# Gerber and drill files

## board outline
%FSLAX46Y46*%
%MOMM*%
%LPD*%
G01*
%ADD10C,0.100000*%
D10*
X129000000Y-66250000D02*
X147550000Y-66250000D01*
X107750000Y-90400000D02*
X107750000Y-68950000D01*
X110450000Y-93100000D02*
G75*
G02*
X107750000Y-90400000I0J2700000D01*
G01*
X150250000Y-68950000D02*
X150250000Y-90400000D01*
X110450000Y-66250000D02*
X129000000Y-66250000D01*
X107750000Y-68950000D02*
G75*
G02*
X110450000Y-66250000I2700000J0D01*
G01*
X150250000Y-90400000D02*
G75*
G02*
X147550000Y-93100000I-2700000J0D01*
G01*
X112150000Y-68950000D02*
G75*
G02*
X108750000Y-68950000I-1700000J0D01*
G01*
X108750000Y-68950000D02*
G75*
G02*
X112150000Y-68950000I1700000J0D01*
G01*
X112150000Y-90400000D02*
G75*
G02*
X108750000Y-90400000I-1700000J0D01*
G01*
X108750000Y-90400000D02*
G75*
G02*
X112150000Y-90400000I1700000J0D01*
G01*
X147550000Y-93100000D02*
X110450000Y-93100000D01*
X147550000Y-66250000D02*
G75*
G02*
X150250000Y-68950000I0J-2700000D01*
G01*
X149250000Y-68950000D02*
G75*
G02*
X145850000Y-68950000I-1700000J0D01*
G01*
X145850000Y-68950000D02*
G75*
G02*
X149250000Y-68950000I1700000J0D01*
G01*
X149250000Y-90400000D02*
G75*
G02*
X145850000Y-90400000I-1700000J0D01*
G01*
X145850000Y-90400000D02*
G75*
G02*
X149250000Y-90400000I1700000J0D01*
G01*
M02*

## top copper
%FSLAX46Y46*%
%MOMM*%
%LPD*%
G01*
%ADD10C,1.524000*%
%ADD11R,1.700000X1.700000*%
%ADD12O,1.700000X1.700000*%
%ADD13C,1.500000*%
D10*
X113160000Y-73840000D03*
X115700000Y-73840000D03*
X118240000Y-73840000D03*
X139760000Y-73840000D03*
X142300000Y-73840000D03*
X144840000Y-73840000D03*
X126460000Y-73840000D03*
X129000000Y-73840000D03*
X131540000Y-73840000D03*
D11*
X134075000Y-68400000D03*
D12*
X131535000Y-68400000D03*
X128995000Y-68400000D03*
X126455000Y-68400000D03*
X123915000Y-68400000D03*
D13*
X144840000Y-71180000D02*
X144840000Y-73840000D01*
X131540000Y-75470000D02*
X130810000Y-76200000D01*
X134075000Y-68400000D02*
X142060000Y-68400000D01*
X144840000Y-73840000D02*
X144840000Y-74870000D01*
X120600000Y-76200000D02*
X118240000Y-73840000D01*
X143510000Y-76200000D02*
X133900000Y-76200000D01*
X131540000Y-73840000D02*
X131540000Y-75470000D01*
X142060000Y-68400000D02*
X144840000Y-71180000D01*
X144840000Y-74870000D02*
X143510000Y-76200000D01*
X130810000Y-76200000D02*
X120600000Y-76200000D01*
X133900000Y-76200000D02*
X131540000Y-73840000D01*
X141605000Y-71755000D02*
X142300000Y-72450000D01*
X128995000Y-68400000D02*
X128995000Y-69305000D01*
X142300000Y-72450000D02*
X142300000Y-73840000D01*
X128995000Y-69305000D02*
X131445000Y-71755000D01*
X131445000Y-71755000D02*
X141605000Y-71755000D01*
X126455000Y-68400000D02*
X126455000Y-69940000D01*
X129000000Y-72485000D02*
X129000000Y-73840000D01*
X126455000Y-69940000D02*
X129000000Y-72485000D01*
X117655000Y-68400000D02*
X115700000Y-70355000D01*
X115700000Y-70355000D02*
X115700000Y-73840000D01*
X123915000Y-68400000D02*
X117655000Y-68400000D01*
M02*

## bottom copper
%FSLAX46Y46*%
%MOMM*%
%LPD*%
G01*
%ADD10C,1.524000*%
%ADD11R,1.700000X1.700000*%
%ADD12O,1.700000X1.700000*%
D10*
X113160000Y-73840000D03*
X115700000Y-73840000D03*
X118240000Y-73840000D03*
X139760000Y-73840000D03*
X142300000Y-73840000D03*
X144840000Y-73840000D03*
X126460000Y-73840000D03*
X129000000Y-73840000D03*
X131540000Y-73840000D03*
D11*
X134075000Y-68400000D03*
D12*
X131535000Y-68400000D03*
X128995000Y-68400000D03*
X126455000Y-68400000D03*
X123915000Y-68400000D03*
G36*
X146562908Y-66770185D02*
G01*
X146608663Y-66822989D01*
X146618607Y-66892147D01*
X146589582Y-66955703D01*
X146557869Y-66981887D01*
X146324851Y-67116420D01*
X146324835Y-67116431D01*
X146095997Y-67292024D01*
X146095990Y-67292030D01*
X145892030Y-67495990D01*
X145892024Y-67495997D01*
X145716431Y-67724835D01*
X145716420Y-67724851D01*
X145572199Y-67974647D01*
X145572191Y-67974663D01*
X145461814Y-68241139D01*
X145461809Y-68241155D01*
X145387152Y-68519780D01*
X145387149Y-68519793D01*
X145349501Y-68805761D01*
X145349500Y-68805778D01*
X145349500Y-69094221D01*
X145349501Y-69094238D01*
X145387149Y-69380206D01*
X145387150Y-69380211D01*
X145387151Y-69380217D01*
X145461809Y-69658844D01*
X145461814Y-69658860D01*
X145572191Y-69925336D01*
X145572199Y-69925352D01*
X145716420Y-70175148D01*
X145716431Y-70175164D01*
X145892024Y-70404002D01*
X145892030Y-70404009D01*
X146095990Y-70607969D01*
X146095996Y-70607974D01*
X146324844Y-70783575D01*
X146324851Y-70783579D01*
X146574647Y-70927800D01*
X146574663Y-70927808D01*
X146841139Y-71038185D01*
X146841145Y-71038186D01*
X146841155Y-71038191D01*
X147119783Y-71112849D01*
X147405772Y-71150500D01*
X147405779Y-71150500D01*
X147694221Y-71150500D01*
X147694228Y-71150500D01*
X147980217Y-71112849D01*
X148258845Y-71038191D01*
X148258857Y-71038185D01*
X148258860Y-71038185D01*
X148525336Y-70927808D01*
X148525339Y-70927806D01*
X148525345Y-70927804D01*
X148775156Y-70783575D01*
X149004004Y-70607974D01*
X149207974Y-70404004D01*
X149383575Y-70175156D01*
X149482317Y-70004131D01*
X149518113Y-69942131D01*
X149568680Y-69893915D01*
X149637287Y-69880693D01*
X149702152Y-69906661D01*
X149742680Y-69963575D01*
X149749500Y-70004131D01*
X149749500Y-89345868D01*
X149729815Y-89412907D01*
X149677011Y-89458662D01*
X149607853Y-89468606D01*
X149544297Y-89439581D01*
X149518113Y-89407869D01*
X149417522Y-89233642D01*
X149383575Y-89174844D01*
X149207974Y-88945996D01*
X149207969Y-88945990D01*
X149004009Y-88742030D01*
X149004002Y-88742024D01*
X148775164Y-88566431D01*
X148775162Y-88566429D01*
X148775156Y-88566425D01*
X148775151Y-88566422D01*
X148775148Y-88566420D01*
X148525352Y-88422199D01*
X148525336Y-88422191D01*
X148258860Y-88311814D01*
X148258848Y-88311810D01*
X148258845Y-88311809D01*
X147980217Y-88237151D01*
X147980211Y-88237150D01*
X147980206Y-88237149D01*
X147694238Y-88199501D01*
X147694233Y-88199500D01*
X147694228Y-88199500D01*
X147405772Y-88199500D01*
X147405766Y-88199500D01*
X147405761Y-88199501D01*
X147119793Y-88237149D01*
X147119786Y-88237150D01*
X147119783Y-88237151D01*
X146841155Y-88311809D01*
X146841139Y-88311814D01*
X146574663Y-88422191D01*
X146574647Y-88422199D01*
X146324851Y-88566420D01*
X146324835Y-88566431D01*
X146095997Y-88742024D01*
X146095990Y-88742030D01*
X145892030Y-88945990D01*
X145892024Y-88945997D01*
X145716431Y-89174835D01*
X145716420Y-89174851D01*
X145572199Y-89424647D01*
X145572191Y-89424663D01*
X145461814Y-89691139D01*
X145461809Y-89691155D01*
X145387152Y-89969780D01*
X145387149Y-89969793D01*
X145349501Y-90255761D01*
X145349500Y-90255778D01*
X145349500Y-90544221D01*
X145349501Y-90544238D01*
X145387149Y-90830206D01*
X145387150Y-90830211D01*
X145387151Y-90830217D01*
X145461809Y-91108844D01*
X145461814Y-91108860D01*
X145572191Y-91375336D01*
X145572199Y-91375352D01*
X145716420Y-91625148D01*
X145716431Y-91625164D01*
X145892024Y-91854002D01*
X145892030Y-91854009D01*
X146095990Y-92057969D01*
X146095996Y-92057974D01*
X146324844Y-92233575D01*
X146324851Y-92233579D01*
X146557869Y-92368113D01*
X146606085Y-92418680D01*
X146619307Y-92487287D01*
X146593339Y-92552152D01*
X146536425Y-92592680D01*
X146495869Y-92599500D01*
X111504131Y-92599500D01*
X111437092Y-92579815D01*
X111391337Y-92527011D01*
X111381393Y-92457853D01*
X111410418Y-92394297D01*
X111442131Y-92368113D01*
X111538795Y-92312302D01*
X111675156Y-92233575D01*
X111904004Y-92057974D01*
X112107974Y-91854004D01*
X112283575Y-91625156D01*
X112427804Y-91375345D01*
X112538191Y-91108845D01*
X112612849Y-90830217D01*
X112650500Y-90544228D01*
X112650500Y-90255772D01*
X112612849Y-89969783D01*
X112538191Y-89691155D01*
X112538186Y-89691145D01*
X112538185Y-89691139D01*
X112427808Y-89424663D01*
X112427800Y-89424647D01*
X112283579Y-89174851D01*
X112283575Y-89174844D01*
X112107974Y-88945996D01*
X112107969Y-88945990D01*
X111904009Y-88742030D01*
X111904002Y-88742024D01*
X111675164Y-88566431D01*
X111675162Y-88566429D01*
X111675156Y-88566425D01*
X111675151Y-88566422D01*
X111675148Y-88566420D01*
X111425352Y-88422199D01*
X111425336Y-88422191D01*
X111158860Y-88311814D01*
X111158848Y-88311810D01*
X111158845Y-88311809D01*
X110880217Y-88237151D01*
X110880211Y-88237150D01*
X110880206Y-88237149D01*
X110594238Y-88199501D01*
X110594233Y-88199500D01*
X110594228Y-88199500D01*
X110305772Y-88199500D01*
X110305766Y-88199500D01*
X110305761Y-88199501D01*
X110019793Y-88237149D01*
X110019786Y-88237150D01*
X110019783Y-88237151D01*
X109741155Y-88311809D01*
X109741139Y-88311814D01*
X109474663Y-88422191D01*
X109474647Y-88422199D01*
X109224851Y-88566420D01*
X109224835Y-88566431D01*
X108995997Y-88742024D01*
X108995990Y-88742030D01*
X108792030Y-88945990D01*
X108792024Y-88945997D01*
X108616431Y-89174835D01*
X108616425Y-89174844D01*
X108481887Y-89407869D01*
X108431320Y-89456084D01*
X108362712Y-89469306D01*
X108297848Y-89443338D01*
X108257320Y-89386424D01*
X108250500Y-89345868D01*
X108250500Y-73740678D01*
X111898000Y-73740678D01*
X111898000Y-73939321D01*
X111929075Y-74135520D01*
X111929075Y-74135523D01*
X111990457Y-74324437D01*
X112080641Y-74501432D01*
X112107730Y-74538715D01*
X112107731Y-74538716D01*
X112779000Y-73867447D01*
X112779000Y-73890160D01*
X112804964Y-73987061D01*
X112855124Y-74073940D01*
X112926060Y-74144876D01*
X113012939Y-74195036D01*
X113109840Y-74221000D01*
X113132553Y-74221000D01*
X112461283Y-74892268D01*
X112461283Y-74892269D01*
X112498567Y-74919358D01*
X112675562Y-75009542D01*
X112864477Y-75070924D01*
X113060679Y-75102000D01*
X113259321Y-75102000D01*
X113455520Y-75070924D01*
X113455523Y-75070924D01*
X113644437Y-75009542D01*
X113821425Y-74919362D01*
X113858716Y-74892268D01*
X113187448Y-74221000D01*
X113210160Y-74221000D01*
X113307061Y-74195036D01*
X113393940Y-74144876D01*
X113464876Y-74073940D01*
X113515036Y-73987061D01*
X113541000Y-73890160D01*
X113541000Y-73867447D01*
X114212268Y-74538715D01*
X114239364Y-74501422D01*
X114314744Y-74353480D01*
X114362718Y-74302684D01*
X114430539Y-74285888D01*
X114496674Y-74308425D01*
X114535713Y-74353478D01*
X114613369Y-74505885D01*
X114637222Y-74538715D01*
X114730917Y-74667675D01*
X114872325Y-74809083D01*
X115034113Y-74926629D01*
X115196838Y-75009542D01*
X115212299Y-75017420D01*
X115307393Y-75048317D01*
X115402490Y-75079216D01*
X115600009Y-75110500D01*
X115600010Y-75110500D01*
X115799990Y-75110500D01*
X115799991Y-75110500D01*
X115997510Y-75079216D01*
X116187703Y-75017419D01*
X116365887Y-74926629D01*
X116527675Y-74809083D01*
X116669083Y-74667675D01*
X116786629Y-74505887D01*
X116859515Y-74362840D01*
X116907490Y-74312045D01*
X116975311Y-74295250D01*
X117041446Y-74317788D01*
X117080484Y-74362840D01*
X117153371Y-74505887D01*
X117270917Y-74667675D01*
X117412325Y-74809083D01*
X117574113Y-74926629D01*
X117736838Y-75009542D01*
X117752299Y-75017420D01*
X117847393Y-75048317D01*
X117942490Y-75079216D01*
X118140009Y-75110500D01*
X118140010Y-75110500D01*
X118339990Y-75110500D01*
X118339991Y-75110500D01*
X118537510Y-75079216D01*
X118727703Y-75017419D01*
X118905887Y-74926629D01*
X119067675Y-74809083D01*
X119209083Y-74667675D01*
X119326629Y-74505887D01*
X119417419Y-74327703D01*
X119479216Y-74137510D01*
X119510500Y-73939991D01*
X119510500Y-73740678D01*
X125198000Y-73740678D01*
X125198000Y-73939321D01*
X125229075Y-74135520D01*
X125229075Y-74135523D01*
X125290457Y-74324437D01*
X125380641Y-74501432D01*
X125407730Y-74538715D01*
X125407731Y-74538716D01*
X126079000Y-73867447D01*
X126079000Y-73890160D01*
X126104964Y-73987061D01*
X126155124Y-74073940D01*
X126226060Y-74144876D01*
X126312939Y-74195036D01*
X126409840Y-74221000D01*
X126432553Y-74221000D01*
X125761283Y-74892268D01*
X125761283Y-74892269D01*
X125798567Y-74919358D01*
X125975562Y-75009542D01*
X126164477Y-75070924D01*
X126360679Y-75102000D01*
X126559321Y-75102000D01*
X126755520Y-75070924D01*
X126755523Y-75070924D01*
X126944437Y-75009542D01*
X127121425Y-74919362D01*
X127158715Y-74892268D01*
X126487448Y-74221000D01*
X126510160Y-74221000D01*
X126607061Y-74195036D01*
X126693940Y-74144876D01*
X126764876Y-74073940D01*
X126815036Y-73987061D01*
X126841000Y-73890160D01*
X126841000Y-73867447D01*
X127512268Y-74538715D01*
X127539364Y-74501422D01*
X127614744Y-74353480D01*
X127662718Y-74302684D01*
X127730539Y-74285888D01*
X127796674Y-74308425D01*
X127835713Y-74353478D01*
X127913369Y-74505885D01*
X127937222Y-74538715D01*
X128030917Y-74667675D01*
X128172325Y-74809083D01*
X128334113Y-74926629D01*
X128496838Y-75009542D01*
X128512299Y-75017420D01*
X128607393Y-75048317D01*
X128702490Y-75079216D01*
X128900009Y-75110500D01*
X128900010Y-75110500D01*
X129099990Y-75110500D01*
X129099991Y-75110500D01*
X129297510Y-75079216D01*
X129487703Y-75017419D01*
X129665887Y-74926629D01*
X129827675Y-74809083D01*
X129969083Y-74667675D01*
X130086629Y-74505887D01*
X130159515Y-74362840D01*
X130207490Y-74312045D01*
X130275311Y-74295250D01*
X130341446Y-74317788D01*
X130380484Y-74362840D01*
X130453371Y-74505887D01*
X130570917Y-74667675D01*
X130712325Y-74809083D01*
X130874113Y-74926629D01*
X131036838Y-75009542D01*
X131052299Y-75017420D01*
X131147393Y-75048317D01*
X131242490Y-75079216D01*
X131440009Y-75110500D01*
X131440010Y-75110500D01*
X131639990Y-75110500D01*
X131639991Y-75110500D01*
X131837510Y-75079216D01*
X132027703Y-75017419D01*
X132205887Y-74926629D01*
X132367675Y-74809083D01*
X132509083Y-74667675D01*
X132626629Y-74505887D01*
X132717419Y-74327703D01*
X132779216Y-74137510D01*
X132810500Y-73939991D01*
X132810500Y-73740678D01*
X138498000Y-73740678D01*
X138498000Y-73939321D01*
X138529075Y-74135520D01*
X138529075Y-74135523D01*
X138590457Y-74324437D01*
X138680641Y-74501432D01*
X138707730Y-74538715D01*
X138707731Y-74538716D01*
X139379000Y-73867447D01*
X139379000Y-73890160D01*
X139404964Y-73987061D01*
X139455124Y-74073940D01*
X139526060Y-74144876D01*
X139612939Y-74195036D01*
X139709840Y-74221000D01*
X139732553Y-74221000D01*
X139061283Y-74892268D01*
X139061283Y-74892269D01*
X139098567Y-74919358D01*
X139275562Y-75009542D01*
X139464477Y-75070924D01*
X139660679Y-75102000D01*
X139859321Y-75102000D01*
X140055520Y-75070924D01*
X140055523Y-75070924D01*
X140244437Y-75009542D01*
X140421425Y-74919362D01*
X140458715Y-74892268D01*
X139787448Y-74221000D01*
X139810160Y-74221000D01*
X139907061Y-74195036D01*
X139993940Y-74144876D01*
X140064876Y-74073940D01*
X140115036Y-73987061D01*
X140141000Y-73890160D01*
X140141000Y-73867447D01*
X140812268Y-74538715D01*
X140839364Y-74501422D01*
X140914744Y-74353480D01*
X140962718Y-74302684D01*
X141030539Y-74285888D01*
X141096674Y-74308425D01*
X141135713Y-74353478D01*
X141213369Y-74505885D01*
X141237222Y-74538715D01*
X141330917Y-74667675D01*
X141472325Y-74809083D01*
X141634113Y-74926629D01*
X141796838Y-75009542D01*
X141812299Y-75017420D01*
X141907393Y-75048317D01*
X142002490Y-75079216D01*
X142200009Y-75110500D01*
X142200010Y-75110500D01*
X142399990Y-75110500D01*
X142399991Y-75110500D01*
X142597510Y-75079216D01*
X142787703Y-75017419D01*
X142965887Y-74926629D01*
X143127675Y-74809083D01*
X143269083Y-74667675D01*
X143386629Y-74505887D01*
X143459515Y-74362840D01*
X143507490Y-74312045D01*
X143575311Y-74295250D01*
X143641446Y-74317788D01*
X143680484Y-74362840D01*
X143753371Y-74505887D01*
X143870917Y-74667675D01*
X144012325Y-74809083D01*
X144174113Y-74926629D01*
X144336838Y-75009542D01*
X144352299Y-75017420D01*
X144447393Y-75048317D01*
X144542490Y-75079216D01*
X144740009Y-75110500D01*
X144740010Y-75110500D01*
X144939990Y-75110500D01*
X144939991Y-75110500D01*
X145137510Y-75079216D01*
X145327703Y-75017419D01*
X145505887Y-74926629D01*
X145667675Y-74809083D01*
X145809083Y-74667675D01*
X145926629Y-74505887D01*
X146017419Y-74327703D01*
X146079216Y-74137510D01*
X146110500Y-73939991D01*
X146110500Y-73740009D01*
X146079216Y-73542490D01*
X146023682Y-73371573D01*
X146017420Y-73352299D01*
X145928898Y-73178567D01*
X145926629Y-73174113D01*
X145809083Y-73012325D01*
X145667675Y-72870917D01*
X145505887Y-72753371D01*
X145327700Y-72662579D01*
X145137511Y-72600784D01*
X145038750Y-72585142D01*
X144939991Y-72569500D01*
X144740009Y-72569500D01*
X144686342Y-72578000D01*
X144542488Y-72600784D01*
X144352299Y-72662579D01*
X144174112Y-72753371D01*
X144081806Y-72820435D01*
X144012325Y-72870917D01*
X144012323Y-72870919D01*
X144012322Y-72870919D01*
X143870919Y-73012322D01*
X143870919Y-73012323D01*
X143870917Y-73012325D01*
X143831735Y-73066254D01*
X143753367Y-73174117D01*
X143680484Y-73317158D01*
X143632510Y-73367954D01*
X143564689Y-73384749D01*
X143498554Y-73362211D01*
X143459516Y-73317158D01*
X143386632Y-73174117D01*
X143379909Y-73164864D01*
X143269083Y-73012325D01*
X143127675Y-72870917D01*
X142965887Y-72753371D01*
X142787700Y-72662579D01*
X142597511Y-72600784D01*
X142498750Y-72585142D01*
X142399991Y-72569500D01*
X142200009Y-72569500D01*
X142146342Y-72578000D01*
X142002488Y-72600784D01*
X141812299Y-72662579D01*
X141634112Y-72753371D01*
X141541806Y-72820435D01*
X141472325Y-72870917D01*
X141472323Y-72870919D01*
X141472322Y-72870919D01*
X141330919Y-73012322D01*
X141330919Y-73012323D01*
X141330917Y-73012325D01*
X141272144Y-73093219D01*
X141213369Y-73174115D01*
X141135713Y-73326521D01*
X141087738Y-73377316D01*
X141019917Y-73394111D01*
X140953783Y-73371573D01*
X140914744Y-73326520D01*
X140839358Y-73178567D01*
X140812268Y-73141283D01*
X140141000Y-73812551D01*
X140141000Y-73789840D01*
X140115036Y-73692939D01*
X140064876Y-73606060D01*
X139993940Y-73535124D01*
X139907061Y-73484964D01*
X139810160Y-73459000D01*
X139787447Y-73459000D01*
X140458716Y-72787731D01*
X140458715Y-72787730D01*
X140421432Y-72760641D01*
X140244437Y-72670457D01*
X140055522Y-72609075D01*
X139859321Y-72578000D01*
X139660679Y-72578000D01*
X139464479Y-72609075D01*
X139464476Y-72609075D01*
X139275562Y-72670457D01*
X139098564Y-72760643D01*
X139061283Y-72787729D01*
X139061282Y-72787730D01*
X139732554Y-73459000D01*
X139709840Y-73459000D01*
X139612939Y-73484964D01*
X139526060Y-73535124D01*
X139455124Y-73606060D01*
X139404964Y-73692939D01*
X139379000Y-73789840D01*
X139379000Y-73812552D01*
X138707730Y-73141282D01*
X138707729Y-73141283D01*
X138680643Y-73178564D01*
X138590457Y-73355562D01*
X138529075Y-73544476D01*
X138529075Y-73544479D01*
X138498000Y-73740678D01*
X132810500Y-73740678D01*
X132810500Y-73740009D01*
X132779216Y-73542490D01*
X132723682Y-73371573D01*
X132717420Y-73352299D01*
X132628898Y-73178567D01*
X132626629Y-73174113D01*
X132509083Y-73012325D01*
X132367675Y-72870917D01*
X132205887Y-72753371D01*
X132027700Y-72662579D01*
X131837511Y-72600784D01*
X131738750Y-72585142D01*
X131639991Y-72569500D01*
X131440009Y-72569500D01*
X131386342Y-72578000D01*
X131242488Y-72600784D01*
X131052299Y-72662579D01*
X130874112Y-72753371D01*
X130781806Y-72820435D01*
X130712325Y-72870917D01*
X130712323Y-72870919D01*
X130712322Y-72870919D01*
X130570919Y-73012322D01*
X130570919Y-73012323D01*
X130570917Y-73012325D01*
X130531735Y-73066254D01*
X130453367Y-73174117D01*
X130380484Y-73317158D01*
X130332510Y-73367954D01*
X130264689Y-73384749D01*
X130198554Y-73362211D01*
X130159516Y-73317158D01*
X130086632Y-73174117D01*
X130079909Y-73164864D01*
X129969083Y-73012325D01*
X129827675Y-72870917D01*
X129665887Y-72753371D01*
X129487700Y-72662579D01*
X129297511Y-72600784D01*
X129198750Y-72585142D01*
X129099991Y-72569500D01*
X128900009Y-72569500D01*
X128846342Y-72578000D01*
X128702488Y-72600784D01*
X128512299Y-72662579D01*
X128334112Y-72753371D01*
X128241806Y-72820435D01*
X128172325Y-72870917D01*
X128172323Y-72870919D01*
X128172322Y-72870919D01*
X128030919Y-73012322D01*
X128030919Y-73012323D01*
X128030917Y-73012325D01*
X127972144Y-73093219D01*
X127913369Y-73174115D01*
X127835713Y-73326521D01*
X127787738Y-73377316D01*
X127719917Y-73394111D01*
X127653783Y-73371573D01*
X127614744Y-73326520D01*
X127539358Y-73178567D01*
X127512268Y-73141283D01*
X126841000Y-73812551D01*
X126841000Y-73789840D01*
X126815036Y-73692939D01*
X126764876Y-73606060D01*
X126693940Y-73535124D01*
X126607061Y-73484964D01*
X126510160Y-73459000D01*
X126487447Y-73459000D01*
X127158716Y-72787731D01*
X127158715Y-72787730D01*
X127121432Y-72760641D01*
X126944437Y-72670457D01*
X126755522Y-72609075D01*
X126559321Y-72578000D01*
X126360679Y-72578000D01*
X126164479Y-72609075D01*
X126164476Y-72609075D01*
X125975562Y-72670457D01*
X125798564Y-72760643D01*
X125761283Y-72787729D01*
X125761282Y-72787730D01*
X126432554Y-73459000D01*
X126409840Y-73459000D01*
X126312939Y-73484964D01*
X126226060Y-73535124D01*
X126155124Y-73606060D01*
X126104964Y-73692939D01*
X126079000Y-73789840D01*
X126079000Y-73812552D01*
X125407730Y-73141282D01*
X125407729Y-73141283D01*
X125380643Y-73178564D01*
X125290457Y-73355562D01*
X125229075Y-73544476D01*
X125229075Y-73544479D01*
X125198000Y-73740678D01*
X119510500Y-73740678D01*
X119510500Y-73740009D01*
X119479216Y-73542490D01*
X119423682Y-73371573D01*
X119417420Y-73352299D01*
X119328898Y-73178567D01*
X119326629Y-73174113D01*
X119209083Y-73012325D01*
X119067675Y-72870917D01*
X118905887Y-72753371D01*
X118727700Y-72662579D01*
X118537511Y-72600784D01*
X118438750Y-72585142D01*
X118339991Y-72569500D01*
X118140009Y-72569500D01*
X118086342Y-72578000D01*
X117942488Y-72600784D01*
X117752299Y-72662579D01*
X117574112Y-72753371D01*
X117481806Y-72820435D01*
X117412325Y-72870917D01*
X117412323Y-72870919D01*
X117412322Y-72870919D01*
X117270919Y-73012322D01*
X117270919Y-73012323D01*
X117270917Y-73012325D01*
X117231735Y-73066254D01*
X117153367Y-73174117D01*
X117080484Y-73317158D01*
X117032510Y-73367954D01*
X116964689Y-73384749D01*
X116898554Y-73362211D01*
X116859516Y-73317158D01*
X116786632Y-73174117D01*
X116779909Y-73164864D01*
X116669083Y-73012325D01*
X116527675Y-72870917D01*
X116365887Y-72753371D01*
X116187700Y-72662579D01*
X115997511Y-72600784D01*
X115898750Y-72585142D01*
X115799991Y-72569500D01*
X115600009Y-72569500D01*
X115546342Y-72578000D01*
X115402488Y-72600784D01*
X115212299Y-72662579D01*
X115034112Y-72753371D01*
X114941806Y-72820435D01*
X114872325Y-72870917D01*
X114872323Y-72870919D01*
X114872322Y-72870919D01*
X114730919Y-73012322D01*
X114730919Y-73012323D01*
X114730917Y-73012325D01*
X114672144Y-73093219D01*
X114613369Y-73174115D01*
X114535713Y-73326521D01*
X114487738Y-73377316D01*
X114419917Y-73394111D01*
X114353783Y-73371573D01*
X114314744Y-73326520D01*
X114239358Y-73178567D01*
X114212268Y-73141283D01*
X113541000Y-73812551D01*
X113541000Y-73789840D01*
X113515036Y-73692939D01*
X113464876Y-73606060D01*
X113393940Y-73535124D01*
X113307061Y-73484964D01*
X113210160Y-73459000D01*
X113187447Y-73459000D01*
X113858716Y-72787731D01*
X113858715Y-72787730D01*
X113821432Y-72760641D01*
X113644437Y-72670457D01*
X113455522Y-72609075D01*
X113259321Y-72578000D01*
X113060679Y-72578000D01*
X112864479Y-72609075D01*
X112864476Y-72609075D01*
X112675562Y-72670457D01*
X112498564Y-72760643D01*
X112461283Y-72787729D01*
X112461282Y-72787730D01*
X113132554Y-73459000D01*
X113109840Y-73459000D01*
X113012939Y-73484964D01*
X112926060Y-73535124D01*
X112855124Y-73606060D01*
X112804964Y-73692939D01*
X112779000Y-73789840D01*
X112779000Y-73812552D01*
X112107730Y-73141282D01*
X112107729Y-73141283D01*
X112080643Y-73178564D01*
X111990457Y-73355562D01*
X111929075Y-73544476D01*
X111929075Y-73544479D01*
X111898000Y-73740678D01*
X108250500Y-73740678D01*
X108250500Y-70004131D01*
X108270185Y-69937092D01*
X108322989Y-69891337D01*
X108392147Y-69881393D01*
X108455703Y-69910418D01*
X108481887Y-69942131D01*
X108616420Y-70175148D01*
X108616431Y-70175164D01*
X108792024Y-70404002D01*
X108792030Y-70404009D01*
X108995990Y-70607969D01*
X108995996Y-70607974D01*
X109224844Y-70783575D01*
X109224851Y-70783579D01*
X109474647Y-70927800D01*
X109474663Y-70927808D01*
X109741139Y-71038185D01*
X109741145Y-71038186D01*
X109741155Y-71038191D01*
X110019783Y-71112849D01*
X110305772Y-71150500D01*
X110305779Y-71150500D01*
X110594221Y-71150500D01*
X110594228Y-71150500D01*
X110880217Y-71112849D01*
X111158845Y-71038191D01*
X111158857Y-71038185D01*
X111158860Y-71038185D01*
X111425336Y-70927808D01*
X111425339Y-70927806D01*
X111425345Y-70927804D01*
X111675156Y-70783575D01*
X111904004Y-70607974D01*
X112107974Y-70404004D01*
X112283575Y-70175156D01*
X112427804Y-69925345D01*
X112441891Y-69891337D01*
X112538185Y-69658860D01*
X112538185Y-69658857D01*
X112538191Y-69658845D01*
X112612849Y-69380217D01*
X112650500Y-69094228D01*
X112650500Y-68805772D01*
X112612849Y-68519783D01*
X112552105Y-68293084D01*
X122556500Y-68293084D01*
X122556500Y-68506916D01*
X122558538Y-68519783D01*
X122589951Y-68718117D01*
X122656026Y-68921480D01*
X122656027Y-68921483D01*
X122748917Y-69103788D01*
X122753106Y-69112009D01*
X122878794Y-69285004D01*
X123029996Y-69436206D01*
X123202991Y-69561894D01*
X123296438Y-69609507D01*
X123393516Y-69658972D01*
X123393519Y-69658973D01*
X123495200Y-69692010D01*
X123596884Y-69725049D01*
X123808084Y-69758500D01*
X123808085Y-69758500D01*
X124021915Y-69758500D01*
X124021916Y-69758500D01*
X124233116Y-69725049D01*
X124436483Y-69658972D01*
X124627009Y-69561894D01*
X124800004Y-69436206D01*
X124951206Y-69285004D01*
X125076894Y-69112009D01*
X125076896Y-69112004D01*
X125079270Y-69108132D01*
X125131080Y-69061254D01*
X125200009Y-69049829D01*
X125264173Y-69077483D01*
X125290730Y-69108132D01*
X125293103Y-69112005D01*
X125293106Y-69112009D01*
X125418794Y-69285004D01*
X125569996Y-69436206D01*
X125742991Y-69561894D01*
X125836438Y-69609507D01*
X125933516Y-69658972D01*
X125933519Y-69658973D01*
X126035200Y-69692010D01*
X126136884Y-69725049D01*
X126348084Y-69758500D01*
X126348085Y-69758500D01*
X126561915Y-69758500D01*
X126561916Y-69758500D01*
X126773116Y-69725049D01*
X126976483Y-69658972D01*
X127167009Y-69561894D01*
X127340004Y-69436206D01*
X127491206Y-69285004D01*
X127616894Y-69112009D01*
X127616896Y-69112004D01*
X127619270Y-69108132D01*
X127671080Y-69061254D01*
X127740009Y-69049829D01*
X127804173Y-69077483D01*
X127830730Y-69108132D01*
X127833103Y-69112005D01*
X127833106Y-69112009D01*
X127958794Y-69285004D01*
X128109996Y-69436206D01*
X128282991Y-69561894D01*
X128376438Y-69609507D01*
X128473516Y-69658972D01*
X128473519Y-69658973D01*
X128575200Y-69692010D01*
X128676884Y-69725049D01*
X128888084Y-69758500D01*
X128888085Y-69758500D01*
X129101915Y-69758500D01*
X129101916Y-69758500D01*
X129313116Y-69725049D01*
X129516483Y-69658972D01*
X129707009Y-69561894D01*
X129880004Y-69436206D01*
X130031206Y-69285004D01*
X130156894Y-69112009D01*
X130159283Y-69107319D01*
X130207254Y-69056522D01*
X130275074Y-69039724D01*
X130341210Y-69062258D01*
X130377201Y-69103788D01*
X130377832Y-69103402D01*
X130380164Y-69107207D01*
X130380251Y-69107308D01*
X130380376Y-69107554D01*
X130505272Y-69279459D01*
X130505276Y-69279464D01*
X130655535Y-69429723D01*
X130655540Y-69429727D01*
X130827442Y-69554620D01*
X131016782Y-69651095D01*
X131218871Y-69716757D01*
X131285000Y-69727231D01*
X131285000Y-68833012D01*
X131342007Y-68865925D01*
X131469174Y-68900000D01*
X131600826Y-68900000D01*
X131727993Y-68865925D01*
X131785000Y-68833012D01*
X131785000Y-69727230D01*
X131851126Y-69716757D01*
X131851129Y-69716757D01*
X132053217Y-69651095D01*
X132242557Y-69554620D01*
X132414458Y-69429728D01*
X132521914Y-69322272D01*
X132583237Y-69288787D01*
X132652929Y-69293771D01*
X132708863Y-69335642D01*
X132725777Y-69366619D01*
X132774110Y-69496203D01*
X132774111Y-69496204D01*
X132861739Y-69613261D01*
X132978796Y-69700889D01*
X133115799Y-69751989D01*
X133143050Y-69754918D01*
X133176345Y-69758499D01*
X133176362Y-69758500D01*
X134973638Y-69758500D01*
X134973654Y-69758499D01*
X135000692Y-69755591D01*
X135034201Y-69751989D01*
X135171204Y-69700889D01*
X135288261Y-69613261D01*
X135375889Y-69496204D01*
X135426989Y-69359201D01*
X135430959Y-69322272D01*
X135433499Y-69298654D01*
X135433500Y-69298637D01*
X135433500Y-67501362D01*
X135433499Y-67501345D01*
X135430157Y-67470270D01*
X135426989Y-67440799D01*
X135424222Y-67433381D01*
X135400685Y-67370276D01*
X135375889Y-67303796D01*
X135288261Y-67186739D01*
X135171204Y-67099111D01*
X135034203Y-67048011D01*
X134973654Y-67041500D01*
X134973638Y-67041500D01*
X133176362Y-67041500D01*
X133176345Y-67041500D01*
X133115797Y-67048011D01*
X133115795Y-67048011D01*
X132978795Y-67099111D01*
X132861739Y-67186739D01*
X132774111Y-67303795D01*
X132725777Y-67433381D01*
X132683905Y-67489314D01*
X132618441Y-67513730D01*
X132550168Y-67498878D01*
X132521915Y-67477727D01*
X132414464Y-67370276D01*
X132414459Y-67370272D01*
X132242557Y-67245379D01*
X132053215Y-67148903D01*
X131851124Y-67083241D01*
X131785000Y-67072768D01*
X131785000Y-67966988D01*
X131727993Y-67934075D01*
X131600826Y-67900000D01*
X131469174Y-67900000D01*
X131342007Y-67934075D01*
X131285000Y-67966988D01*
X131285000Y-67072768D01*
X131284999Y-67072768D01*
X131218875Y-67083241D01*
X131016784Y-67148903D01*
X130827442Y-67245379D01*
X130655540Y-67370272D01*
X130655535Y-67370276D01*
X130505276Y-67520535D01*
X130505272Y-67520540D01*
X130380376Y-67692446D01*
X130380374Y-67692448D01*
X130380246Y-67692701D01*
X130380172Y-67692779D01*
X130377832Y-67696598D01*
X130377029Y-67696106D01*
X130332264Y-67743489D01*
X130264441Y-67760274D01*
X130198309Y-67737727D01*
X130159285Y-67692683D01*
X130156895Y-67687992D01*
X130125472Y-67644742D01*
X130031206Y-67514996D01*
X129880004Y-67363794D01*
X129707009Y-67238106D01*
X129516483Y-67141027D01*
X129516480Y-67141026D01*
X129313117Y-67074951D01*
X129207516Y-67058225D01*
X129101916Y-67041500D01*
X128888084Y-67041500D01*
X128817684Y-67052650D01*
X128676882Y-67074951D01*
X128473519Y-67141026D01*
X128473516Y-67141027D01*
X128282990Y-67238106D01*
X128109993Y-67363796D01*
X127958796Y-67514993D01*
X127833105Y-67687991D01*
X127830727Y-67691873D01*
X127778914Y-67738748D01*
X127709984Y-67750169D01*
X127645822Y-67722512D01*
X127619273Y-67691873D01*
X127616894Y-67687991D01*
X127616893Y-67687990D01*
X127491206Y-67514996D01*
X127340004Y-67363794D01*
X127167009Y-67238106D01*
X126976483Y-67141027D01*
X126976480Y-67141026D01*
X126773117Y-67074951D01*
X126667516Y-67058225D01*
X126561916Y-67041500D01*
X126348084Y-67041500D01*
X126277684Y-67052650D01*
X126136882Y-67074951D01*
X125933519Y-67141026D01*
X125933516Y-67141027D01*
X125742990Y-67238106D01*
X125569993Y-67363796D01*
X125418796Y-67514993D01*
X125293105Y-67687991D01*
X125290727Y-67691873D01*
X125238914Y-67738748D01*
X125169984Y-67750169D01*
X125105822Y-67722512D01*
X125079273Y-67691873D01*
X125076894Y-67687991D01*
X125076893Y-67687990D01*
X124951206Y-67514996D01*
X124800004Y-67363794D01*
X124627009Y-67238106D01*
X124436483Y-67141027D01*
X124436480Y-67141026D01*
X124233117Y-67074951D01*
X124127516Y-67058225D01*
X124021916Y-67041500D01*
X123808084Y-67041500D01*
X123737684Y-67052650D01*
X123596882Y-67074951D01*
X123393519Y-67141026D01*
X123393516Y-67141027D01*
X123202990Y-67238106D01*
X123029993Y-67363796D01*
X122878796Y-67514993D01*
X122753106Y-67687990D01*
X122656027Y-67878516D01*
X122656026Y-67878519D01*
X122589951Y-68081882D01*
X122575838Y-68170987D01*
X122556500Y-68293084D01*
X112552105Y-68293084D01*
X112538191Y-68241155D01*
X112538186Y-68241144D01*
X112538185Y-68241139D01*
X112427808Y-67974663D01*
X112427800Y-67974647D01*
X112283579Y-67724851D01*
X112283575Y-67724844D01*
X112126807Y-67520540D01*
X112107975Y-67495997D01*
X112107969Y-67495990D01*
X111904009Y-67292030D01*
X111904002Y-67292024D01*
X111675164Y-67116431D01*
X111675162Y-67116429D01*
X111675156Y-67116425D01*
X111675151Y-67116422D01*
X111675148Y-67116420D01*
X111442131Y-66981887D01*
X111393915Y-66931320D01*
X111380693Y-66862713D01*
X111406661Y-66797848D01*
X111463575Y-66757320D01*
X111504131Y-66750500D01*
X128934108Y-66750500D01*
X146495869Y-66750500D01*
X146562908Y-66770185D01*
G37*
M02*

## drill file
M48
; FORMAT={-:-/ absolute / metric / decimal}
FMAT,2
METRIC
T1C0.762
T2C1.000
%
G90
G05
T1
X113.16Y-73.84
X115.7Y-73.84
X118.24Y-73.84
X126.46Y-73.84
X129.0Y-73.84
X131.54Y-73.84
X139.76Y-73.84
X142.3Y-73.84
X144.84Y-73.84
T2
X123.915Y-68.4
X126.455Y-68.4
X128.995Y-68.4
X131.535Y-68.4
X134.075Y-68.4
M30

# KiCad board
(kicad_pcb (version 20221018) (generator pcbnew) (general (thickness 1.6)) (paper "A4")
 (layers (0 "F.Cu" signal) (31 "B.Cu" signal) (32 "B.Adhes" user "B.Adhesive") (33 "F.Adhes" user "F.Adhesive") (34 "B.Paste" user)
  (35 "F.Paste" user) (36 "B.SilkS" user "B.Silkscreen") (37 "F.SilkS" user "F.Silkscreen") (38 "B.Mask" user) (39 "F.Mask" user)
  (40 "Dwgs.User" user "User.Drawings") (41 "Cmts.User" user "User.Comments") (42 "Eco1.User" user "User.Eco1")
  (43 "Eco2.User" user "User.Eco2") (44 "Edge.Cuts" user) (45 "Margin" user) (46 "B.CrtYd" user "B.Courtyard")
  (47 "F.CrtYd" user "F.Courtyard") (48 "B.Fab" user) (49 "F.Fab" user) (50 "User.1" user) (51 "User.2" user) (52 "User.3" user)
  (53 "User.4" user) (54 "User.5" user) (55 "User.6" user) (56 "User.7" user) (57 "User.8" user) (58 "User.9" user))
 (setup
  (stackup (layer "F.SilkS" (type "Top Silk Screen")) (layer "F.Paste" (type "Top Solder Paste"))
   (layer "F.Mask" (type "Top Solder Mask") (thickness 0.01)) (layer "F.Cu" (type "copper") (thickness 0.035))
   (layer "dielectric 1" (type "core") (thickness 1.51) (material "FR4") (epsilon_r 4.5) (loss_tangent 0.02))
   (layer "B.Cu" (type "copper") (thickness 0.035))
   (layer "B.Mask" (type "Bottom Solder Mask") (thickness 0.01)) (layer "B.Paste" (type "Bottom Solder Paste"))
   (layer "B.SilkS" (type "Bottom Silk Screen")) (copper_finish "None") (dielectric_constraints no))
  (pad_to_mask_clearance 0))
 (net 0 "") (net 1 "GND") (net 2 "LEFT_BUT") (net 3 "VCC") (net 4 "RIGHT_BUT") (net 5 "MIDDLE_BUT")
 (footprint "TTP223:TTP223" (layer "F.Cu") (at 115.7 79)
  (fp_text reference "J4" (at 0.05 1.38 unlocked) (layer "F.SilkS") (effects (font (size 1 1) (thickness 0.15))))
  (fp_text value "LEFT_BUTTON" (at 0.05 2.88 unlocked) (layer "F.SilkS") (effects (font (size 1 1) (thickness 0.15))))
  (pad "1" thru_hole circle (at -2.54 -5.16) (size 1.524 1.524) (drill 0.762) (layers "*.Cu" "*.Mask") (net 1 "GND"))
  (pad "2" thru_hole circle (at 0 -5.16) (size 1.524 1.524) (drill 0.762) (layers "*.Cu" "*.Mask") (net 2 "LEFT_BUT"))
  (pad "3" thru_hole circle (at 2.54 -5.16) (size 1.524 1.524) (drill 0.762) (layers "*.Cu" "*.Mask") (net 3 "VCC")))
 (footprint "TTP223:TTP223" (layer "F.Cu") (at 142.3 79)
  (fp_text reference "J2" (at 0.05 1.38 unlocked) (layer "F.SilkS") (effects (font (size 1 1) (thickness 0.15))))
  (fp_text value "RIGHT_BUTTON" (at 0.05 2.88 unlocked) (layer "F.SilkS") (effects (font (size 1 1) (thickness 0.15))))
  (pad "1" thru_hole circle (at -2.54 -5.16) (size 1.524 1.524) (drill 0.762) (layers "*.Cu" "*.Mask") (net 1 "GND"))
  (pad "2" thru_hole circle (at 0 -5.16) (size 1.524 1.524) (drill 0.762) (layers "*.Cu" "*.Mask") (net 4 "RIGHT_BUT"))
  (pad "3" thru_hole circle (at 2.54 -5.16) (size 1.524 1.524) (drill 0.762) (layers "*.Cu" "*.Mask") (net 3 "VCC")))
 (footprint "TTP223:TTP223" (layer "F.Cu") (at 129 79)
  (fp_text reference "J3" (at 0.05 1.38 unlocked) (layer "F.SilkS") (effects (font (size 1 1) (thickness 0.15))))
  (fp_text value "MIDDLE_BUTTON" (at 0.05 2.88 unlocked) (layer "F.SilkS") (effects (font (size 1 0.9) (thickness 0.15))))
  (pad "1" thru_hole circle (at -2.54 -5.16) (size 1.524 1.524) (drill 0.762) (layers "*.Cu" "*.Mask") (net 1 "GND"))
  (pad "2" thru_hole circle (at 0 -5.16) (size 1.524 1.524) (drill 0.762) (layers "*.Cu" "*.Mask") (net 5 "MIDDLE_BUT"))
  (pad "3" thru_hole circle (at 2.54 -5.16) (size 1.524 1.524) (drill 0.762) (layers "*.Cu" "*.Mask") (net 3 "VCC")))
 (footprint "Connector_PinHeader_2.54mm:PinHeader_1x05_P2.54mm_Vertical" (layer "B.Cu") (at 134.075 68.4 90)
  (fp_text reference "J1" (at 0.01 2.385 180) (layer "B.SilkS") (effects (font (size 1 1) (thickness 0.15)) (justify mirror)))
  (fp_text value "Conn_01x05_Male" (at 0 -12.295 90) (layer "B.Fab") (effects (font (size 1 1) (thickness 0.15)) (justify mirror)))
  (pad "1" thru_hole rect (at 0 0 90) (size 1.7 1.7) (drill 1) (layers "*.Cu" "*.Mask") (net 3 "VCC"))
  (pad "2" thru_hole oval (at 0 -2.54 90) (size 1.7 1.7) (drill 1) (layers "*.Cu" "*.Mask") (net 1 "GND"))
  (pad "3" thru_hole oval (at 0 -5.08 90) (size 1.7 1.7) (drill 1) (layers "*.Cu" "*.Mask") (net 4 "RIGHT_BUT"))
  (pad "4" thru_hole oval (at 0 -7.62 90) (size 1.7 1.7) (drill 1) (layers "*.Cu" "*.Mask") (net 5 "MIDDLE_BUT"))
  (pad "5" thru_hole oval (at 0 -10.16 90) (size 1.7 1.7) (drill 1) (layers "*.Cu" "*.Mask") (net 2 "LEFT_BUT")))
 (gr_line (start 129 66.25) (end 147.55 66.25) (stroke (width 0.1) (type solid)) (layer "Edge.Cuts"))
 (gr_line (start 107.75 90.4) (end 107.75 68.95) (stroke (width 0.1) (type solid)) (layer "Edge.Cuts"))
 (gr_arc (start 110.45 93.1) (mid 108.540812 92.309188) (end 107.75 90.4) (stroke (width 0.1) (type solid)) (layer "Edge.Cuts"))
 (gr_line (start 150.25 68.95) (end 150.25 90.4) (stroke (width 0.1) (type solid)) (layer "Edge.Cuts"))
 (gr_line (start 110.45 66.25) (end 129 66.25) (stroke (width 0.1) (type solid)) (layer "Edge.Cuts"))
 (gr_arc (start 107.75 68.95) (mid 108.540812 67.040812) (end 110.45 66.25) (stroke (width 0.1) (type solid)) (layer "Edge.Cuts"))
 (gr_arc (start 150.25 90.4) (mid 149.459188 92.309188) (end 147.55 93.1) (stroke (width 0.1) (type solid)) (layer "Edge.Cuts"))
 (gr_circle (center 110.45 68.95) (end 112.15 68.95) (stroke (width 0.1) (type solid)) (fill none) (layer "Edge.Cuts"))
 (gr_circle (center 110.45 90.4) (end 112.15 90.4) (stroke (width 0.1) (type solid)) (fill none) (layer "Edge.Cuts"))
 (gr_line (start 147.55 93.1) (end 110.45 93.1) (stroke (width 0.1) (type solid)) (layer "Edge.Cuts"))
 (gr_arc (start 147.55 66.25) (mid 149.459188 67.040812) (end 150.25 68.95) (stroke (width 0.1) (type solid)) (layer "Edge.Cuts"))
 (gr_circle (center 147.55 68.95) (end 149.25 68.95) (stroke (width 0.1) (type solid)) (fill none) (layer "Edge.Cuts"))
 (gr_circle (center 147.55 90.4) (end 149.25 90.4) (stroke (width 0.1) (type solid)) (fill none) (layer "Edge.Cuts"))
 (segment (start 144.84 71.18) (end 144.84 73.84) (width 1.5) (layer "F.Cu") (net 3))
 (segment (start 131.54 75.47) (end 130.81 76.2) (width 1.5) (layer "F.Cu") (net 3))
 (segment (start 134.075 68.4) (end 142.06 68.4) (width 1.5) (layer "F.Cu") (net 3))
 (segment (start 144.84 73.84) (end 144.84 74.87) (width 1.5) (layer "F.Cu") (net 3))
 (segment (start 120.6 76.2) (end 118.24 73.84) (width 1.5) (layer "F.Cu") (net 3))
 (segment (start 143.51 76.2) (end 133.9 76.2) (width 1.5) (layer "F.Cu") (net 3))
 (segment (start 131.54 73.84) (end 131.54 75.47) (width 1.5) (layer "F.Cu") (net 3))
 (segment (start 142.06 68.4) (end 144.84 71.18) (width 1.5) (layer "F.Cu") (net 3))
 (segment (start 144.84 74.87) (end 143.51 76.2) (width 1.5) (layer "F.Cu") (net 3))
 (segment (start 130.81 76.2) (end 120.6 76.2) (width 1.5) (layer "F.Cu") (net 3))
 (segment (start 133.9 76.2) (end 131.54 73.84) (width 1.5) (layer "F.Cu") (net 3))
 (segment (start 141.605 71.755) (end 142.3 72.45) (width 1.5) (layer "F.Cu") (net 4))
 (segment (start 128.995 68.4) (end 128.995 69.305) (width 1.5) (layer "F.Cu") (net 4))
 (segment (start 142.3 72.45) (end 142.3 73.84) (width 1.5) (layer "F.Cu") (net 4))
 (segment (start 128.995 69.305) (end 131.445 71.755) (width 1.5) (layer "F.Cu") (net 4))
 (segment (start 131.445 71.755) (end 141.605 71.755) (width 1.5) (layer "F.Cu") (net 4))
 (segment (start 126.455 68.4) (end 126.455 69.94) (width 1.5) (layer "F.Cu") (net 5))
 (segment (start 129 72.485) (end 129 73.84) (width 1.5) (layer "F.Cu") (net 5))
 (segment (start 126.455 69.94) (end 129 72.485) (width 1.5) (layer "F.Cu") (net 5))
 (segment (start 117.655 68.4) (end 115.7 70.355) (width 1.5) (layer "F.Cu") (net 2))
 (segment (start 115.7 70.355) (end 115.7 73.84) (width 1.5) (layer "F.Cu") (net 2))
 (segment (start 123.915 68.4) (end 117.655 68.4) (width 1.5) (layer "F.Cu") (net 2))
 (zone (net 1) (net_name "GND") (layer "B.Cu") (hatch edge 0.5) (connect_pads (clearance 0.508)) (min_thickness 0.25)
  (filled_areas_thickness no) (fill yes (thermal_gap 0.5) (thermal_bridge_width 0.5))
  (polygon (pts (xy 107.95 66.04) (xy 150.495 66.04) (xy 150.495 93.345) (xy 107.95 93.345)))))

